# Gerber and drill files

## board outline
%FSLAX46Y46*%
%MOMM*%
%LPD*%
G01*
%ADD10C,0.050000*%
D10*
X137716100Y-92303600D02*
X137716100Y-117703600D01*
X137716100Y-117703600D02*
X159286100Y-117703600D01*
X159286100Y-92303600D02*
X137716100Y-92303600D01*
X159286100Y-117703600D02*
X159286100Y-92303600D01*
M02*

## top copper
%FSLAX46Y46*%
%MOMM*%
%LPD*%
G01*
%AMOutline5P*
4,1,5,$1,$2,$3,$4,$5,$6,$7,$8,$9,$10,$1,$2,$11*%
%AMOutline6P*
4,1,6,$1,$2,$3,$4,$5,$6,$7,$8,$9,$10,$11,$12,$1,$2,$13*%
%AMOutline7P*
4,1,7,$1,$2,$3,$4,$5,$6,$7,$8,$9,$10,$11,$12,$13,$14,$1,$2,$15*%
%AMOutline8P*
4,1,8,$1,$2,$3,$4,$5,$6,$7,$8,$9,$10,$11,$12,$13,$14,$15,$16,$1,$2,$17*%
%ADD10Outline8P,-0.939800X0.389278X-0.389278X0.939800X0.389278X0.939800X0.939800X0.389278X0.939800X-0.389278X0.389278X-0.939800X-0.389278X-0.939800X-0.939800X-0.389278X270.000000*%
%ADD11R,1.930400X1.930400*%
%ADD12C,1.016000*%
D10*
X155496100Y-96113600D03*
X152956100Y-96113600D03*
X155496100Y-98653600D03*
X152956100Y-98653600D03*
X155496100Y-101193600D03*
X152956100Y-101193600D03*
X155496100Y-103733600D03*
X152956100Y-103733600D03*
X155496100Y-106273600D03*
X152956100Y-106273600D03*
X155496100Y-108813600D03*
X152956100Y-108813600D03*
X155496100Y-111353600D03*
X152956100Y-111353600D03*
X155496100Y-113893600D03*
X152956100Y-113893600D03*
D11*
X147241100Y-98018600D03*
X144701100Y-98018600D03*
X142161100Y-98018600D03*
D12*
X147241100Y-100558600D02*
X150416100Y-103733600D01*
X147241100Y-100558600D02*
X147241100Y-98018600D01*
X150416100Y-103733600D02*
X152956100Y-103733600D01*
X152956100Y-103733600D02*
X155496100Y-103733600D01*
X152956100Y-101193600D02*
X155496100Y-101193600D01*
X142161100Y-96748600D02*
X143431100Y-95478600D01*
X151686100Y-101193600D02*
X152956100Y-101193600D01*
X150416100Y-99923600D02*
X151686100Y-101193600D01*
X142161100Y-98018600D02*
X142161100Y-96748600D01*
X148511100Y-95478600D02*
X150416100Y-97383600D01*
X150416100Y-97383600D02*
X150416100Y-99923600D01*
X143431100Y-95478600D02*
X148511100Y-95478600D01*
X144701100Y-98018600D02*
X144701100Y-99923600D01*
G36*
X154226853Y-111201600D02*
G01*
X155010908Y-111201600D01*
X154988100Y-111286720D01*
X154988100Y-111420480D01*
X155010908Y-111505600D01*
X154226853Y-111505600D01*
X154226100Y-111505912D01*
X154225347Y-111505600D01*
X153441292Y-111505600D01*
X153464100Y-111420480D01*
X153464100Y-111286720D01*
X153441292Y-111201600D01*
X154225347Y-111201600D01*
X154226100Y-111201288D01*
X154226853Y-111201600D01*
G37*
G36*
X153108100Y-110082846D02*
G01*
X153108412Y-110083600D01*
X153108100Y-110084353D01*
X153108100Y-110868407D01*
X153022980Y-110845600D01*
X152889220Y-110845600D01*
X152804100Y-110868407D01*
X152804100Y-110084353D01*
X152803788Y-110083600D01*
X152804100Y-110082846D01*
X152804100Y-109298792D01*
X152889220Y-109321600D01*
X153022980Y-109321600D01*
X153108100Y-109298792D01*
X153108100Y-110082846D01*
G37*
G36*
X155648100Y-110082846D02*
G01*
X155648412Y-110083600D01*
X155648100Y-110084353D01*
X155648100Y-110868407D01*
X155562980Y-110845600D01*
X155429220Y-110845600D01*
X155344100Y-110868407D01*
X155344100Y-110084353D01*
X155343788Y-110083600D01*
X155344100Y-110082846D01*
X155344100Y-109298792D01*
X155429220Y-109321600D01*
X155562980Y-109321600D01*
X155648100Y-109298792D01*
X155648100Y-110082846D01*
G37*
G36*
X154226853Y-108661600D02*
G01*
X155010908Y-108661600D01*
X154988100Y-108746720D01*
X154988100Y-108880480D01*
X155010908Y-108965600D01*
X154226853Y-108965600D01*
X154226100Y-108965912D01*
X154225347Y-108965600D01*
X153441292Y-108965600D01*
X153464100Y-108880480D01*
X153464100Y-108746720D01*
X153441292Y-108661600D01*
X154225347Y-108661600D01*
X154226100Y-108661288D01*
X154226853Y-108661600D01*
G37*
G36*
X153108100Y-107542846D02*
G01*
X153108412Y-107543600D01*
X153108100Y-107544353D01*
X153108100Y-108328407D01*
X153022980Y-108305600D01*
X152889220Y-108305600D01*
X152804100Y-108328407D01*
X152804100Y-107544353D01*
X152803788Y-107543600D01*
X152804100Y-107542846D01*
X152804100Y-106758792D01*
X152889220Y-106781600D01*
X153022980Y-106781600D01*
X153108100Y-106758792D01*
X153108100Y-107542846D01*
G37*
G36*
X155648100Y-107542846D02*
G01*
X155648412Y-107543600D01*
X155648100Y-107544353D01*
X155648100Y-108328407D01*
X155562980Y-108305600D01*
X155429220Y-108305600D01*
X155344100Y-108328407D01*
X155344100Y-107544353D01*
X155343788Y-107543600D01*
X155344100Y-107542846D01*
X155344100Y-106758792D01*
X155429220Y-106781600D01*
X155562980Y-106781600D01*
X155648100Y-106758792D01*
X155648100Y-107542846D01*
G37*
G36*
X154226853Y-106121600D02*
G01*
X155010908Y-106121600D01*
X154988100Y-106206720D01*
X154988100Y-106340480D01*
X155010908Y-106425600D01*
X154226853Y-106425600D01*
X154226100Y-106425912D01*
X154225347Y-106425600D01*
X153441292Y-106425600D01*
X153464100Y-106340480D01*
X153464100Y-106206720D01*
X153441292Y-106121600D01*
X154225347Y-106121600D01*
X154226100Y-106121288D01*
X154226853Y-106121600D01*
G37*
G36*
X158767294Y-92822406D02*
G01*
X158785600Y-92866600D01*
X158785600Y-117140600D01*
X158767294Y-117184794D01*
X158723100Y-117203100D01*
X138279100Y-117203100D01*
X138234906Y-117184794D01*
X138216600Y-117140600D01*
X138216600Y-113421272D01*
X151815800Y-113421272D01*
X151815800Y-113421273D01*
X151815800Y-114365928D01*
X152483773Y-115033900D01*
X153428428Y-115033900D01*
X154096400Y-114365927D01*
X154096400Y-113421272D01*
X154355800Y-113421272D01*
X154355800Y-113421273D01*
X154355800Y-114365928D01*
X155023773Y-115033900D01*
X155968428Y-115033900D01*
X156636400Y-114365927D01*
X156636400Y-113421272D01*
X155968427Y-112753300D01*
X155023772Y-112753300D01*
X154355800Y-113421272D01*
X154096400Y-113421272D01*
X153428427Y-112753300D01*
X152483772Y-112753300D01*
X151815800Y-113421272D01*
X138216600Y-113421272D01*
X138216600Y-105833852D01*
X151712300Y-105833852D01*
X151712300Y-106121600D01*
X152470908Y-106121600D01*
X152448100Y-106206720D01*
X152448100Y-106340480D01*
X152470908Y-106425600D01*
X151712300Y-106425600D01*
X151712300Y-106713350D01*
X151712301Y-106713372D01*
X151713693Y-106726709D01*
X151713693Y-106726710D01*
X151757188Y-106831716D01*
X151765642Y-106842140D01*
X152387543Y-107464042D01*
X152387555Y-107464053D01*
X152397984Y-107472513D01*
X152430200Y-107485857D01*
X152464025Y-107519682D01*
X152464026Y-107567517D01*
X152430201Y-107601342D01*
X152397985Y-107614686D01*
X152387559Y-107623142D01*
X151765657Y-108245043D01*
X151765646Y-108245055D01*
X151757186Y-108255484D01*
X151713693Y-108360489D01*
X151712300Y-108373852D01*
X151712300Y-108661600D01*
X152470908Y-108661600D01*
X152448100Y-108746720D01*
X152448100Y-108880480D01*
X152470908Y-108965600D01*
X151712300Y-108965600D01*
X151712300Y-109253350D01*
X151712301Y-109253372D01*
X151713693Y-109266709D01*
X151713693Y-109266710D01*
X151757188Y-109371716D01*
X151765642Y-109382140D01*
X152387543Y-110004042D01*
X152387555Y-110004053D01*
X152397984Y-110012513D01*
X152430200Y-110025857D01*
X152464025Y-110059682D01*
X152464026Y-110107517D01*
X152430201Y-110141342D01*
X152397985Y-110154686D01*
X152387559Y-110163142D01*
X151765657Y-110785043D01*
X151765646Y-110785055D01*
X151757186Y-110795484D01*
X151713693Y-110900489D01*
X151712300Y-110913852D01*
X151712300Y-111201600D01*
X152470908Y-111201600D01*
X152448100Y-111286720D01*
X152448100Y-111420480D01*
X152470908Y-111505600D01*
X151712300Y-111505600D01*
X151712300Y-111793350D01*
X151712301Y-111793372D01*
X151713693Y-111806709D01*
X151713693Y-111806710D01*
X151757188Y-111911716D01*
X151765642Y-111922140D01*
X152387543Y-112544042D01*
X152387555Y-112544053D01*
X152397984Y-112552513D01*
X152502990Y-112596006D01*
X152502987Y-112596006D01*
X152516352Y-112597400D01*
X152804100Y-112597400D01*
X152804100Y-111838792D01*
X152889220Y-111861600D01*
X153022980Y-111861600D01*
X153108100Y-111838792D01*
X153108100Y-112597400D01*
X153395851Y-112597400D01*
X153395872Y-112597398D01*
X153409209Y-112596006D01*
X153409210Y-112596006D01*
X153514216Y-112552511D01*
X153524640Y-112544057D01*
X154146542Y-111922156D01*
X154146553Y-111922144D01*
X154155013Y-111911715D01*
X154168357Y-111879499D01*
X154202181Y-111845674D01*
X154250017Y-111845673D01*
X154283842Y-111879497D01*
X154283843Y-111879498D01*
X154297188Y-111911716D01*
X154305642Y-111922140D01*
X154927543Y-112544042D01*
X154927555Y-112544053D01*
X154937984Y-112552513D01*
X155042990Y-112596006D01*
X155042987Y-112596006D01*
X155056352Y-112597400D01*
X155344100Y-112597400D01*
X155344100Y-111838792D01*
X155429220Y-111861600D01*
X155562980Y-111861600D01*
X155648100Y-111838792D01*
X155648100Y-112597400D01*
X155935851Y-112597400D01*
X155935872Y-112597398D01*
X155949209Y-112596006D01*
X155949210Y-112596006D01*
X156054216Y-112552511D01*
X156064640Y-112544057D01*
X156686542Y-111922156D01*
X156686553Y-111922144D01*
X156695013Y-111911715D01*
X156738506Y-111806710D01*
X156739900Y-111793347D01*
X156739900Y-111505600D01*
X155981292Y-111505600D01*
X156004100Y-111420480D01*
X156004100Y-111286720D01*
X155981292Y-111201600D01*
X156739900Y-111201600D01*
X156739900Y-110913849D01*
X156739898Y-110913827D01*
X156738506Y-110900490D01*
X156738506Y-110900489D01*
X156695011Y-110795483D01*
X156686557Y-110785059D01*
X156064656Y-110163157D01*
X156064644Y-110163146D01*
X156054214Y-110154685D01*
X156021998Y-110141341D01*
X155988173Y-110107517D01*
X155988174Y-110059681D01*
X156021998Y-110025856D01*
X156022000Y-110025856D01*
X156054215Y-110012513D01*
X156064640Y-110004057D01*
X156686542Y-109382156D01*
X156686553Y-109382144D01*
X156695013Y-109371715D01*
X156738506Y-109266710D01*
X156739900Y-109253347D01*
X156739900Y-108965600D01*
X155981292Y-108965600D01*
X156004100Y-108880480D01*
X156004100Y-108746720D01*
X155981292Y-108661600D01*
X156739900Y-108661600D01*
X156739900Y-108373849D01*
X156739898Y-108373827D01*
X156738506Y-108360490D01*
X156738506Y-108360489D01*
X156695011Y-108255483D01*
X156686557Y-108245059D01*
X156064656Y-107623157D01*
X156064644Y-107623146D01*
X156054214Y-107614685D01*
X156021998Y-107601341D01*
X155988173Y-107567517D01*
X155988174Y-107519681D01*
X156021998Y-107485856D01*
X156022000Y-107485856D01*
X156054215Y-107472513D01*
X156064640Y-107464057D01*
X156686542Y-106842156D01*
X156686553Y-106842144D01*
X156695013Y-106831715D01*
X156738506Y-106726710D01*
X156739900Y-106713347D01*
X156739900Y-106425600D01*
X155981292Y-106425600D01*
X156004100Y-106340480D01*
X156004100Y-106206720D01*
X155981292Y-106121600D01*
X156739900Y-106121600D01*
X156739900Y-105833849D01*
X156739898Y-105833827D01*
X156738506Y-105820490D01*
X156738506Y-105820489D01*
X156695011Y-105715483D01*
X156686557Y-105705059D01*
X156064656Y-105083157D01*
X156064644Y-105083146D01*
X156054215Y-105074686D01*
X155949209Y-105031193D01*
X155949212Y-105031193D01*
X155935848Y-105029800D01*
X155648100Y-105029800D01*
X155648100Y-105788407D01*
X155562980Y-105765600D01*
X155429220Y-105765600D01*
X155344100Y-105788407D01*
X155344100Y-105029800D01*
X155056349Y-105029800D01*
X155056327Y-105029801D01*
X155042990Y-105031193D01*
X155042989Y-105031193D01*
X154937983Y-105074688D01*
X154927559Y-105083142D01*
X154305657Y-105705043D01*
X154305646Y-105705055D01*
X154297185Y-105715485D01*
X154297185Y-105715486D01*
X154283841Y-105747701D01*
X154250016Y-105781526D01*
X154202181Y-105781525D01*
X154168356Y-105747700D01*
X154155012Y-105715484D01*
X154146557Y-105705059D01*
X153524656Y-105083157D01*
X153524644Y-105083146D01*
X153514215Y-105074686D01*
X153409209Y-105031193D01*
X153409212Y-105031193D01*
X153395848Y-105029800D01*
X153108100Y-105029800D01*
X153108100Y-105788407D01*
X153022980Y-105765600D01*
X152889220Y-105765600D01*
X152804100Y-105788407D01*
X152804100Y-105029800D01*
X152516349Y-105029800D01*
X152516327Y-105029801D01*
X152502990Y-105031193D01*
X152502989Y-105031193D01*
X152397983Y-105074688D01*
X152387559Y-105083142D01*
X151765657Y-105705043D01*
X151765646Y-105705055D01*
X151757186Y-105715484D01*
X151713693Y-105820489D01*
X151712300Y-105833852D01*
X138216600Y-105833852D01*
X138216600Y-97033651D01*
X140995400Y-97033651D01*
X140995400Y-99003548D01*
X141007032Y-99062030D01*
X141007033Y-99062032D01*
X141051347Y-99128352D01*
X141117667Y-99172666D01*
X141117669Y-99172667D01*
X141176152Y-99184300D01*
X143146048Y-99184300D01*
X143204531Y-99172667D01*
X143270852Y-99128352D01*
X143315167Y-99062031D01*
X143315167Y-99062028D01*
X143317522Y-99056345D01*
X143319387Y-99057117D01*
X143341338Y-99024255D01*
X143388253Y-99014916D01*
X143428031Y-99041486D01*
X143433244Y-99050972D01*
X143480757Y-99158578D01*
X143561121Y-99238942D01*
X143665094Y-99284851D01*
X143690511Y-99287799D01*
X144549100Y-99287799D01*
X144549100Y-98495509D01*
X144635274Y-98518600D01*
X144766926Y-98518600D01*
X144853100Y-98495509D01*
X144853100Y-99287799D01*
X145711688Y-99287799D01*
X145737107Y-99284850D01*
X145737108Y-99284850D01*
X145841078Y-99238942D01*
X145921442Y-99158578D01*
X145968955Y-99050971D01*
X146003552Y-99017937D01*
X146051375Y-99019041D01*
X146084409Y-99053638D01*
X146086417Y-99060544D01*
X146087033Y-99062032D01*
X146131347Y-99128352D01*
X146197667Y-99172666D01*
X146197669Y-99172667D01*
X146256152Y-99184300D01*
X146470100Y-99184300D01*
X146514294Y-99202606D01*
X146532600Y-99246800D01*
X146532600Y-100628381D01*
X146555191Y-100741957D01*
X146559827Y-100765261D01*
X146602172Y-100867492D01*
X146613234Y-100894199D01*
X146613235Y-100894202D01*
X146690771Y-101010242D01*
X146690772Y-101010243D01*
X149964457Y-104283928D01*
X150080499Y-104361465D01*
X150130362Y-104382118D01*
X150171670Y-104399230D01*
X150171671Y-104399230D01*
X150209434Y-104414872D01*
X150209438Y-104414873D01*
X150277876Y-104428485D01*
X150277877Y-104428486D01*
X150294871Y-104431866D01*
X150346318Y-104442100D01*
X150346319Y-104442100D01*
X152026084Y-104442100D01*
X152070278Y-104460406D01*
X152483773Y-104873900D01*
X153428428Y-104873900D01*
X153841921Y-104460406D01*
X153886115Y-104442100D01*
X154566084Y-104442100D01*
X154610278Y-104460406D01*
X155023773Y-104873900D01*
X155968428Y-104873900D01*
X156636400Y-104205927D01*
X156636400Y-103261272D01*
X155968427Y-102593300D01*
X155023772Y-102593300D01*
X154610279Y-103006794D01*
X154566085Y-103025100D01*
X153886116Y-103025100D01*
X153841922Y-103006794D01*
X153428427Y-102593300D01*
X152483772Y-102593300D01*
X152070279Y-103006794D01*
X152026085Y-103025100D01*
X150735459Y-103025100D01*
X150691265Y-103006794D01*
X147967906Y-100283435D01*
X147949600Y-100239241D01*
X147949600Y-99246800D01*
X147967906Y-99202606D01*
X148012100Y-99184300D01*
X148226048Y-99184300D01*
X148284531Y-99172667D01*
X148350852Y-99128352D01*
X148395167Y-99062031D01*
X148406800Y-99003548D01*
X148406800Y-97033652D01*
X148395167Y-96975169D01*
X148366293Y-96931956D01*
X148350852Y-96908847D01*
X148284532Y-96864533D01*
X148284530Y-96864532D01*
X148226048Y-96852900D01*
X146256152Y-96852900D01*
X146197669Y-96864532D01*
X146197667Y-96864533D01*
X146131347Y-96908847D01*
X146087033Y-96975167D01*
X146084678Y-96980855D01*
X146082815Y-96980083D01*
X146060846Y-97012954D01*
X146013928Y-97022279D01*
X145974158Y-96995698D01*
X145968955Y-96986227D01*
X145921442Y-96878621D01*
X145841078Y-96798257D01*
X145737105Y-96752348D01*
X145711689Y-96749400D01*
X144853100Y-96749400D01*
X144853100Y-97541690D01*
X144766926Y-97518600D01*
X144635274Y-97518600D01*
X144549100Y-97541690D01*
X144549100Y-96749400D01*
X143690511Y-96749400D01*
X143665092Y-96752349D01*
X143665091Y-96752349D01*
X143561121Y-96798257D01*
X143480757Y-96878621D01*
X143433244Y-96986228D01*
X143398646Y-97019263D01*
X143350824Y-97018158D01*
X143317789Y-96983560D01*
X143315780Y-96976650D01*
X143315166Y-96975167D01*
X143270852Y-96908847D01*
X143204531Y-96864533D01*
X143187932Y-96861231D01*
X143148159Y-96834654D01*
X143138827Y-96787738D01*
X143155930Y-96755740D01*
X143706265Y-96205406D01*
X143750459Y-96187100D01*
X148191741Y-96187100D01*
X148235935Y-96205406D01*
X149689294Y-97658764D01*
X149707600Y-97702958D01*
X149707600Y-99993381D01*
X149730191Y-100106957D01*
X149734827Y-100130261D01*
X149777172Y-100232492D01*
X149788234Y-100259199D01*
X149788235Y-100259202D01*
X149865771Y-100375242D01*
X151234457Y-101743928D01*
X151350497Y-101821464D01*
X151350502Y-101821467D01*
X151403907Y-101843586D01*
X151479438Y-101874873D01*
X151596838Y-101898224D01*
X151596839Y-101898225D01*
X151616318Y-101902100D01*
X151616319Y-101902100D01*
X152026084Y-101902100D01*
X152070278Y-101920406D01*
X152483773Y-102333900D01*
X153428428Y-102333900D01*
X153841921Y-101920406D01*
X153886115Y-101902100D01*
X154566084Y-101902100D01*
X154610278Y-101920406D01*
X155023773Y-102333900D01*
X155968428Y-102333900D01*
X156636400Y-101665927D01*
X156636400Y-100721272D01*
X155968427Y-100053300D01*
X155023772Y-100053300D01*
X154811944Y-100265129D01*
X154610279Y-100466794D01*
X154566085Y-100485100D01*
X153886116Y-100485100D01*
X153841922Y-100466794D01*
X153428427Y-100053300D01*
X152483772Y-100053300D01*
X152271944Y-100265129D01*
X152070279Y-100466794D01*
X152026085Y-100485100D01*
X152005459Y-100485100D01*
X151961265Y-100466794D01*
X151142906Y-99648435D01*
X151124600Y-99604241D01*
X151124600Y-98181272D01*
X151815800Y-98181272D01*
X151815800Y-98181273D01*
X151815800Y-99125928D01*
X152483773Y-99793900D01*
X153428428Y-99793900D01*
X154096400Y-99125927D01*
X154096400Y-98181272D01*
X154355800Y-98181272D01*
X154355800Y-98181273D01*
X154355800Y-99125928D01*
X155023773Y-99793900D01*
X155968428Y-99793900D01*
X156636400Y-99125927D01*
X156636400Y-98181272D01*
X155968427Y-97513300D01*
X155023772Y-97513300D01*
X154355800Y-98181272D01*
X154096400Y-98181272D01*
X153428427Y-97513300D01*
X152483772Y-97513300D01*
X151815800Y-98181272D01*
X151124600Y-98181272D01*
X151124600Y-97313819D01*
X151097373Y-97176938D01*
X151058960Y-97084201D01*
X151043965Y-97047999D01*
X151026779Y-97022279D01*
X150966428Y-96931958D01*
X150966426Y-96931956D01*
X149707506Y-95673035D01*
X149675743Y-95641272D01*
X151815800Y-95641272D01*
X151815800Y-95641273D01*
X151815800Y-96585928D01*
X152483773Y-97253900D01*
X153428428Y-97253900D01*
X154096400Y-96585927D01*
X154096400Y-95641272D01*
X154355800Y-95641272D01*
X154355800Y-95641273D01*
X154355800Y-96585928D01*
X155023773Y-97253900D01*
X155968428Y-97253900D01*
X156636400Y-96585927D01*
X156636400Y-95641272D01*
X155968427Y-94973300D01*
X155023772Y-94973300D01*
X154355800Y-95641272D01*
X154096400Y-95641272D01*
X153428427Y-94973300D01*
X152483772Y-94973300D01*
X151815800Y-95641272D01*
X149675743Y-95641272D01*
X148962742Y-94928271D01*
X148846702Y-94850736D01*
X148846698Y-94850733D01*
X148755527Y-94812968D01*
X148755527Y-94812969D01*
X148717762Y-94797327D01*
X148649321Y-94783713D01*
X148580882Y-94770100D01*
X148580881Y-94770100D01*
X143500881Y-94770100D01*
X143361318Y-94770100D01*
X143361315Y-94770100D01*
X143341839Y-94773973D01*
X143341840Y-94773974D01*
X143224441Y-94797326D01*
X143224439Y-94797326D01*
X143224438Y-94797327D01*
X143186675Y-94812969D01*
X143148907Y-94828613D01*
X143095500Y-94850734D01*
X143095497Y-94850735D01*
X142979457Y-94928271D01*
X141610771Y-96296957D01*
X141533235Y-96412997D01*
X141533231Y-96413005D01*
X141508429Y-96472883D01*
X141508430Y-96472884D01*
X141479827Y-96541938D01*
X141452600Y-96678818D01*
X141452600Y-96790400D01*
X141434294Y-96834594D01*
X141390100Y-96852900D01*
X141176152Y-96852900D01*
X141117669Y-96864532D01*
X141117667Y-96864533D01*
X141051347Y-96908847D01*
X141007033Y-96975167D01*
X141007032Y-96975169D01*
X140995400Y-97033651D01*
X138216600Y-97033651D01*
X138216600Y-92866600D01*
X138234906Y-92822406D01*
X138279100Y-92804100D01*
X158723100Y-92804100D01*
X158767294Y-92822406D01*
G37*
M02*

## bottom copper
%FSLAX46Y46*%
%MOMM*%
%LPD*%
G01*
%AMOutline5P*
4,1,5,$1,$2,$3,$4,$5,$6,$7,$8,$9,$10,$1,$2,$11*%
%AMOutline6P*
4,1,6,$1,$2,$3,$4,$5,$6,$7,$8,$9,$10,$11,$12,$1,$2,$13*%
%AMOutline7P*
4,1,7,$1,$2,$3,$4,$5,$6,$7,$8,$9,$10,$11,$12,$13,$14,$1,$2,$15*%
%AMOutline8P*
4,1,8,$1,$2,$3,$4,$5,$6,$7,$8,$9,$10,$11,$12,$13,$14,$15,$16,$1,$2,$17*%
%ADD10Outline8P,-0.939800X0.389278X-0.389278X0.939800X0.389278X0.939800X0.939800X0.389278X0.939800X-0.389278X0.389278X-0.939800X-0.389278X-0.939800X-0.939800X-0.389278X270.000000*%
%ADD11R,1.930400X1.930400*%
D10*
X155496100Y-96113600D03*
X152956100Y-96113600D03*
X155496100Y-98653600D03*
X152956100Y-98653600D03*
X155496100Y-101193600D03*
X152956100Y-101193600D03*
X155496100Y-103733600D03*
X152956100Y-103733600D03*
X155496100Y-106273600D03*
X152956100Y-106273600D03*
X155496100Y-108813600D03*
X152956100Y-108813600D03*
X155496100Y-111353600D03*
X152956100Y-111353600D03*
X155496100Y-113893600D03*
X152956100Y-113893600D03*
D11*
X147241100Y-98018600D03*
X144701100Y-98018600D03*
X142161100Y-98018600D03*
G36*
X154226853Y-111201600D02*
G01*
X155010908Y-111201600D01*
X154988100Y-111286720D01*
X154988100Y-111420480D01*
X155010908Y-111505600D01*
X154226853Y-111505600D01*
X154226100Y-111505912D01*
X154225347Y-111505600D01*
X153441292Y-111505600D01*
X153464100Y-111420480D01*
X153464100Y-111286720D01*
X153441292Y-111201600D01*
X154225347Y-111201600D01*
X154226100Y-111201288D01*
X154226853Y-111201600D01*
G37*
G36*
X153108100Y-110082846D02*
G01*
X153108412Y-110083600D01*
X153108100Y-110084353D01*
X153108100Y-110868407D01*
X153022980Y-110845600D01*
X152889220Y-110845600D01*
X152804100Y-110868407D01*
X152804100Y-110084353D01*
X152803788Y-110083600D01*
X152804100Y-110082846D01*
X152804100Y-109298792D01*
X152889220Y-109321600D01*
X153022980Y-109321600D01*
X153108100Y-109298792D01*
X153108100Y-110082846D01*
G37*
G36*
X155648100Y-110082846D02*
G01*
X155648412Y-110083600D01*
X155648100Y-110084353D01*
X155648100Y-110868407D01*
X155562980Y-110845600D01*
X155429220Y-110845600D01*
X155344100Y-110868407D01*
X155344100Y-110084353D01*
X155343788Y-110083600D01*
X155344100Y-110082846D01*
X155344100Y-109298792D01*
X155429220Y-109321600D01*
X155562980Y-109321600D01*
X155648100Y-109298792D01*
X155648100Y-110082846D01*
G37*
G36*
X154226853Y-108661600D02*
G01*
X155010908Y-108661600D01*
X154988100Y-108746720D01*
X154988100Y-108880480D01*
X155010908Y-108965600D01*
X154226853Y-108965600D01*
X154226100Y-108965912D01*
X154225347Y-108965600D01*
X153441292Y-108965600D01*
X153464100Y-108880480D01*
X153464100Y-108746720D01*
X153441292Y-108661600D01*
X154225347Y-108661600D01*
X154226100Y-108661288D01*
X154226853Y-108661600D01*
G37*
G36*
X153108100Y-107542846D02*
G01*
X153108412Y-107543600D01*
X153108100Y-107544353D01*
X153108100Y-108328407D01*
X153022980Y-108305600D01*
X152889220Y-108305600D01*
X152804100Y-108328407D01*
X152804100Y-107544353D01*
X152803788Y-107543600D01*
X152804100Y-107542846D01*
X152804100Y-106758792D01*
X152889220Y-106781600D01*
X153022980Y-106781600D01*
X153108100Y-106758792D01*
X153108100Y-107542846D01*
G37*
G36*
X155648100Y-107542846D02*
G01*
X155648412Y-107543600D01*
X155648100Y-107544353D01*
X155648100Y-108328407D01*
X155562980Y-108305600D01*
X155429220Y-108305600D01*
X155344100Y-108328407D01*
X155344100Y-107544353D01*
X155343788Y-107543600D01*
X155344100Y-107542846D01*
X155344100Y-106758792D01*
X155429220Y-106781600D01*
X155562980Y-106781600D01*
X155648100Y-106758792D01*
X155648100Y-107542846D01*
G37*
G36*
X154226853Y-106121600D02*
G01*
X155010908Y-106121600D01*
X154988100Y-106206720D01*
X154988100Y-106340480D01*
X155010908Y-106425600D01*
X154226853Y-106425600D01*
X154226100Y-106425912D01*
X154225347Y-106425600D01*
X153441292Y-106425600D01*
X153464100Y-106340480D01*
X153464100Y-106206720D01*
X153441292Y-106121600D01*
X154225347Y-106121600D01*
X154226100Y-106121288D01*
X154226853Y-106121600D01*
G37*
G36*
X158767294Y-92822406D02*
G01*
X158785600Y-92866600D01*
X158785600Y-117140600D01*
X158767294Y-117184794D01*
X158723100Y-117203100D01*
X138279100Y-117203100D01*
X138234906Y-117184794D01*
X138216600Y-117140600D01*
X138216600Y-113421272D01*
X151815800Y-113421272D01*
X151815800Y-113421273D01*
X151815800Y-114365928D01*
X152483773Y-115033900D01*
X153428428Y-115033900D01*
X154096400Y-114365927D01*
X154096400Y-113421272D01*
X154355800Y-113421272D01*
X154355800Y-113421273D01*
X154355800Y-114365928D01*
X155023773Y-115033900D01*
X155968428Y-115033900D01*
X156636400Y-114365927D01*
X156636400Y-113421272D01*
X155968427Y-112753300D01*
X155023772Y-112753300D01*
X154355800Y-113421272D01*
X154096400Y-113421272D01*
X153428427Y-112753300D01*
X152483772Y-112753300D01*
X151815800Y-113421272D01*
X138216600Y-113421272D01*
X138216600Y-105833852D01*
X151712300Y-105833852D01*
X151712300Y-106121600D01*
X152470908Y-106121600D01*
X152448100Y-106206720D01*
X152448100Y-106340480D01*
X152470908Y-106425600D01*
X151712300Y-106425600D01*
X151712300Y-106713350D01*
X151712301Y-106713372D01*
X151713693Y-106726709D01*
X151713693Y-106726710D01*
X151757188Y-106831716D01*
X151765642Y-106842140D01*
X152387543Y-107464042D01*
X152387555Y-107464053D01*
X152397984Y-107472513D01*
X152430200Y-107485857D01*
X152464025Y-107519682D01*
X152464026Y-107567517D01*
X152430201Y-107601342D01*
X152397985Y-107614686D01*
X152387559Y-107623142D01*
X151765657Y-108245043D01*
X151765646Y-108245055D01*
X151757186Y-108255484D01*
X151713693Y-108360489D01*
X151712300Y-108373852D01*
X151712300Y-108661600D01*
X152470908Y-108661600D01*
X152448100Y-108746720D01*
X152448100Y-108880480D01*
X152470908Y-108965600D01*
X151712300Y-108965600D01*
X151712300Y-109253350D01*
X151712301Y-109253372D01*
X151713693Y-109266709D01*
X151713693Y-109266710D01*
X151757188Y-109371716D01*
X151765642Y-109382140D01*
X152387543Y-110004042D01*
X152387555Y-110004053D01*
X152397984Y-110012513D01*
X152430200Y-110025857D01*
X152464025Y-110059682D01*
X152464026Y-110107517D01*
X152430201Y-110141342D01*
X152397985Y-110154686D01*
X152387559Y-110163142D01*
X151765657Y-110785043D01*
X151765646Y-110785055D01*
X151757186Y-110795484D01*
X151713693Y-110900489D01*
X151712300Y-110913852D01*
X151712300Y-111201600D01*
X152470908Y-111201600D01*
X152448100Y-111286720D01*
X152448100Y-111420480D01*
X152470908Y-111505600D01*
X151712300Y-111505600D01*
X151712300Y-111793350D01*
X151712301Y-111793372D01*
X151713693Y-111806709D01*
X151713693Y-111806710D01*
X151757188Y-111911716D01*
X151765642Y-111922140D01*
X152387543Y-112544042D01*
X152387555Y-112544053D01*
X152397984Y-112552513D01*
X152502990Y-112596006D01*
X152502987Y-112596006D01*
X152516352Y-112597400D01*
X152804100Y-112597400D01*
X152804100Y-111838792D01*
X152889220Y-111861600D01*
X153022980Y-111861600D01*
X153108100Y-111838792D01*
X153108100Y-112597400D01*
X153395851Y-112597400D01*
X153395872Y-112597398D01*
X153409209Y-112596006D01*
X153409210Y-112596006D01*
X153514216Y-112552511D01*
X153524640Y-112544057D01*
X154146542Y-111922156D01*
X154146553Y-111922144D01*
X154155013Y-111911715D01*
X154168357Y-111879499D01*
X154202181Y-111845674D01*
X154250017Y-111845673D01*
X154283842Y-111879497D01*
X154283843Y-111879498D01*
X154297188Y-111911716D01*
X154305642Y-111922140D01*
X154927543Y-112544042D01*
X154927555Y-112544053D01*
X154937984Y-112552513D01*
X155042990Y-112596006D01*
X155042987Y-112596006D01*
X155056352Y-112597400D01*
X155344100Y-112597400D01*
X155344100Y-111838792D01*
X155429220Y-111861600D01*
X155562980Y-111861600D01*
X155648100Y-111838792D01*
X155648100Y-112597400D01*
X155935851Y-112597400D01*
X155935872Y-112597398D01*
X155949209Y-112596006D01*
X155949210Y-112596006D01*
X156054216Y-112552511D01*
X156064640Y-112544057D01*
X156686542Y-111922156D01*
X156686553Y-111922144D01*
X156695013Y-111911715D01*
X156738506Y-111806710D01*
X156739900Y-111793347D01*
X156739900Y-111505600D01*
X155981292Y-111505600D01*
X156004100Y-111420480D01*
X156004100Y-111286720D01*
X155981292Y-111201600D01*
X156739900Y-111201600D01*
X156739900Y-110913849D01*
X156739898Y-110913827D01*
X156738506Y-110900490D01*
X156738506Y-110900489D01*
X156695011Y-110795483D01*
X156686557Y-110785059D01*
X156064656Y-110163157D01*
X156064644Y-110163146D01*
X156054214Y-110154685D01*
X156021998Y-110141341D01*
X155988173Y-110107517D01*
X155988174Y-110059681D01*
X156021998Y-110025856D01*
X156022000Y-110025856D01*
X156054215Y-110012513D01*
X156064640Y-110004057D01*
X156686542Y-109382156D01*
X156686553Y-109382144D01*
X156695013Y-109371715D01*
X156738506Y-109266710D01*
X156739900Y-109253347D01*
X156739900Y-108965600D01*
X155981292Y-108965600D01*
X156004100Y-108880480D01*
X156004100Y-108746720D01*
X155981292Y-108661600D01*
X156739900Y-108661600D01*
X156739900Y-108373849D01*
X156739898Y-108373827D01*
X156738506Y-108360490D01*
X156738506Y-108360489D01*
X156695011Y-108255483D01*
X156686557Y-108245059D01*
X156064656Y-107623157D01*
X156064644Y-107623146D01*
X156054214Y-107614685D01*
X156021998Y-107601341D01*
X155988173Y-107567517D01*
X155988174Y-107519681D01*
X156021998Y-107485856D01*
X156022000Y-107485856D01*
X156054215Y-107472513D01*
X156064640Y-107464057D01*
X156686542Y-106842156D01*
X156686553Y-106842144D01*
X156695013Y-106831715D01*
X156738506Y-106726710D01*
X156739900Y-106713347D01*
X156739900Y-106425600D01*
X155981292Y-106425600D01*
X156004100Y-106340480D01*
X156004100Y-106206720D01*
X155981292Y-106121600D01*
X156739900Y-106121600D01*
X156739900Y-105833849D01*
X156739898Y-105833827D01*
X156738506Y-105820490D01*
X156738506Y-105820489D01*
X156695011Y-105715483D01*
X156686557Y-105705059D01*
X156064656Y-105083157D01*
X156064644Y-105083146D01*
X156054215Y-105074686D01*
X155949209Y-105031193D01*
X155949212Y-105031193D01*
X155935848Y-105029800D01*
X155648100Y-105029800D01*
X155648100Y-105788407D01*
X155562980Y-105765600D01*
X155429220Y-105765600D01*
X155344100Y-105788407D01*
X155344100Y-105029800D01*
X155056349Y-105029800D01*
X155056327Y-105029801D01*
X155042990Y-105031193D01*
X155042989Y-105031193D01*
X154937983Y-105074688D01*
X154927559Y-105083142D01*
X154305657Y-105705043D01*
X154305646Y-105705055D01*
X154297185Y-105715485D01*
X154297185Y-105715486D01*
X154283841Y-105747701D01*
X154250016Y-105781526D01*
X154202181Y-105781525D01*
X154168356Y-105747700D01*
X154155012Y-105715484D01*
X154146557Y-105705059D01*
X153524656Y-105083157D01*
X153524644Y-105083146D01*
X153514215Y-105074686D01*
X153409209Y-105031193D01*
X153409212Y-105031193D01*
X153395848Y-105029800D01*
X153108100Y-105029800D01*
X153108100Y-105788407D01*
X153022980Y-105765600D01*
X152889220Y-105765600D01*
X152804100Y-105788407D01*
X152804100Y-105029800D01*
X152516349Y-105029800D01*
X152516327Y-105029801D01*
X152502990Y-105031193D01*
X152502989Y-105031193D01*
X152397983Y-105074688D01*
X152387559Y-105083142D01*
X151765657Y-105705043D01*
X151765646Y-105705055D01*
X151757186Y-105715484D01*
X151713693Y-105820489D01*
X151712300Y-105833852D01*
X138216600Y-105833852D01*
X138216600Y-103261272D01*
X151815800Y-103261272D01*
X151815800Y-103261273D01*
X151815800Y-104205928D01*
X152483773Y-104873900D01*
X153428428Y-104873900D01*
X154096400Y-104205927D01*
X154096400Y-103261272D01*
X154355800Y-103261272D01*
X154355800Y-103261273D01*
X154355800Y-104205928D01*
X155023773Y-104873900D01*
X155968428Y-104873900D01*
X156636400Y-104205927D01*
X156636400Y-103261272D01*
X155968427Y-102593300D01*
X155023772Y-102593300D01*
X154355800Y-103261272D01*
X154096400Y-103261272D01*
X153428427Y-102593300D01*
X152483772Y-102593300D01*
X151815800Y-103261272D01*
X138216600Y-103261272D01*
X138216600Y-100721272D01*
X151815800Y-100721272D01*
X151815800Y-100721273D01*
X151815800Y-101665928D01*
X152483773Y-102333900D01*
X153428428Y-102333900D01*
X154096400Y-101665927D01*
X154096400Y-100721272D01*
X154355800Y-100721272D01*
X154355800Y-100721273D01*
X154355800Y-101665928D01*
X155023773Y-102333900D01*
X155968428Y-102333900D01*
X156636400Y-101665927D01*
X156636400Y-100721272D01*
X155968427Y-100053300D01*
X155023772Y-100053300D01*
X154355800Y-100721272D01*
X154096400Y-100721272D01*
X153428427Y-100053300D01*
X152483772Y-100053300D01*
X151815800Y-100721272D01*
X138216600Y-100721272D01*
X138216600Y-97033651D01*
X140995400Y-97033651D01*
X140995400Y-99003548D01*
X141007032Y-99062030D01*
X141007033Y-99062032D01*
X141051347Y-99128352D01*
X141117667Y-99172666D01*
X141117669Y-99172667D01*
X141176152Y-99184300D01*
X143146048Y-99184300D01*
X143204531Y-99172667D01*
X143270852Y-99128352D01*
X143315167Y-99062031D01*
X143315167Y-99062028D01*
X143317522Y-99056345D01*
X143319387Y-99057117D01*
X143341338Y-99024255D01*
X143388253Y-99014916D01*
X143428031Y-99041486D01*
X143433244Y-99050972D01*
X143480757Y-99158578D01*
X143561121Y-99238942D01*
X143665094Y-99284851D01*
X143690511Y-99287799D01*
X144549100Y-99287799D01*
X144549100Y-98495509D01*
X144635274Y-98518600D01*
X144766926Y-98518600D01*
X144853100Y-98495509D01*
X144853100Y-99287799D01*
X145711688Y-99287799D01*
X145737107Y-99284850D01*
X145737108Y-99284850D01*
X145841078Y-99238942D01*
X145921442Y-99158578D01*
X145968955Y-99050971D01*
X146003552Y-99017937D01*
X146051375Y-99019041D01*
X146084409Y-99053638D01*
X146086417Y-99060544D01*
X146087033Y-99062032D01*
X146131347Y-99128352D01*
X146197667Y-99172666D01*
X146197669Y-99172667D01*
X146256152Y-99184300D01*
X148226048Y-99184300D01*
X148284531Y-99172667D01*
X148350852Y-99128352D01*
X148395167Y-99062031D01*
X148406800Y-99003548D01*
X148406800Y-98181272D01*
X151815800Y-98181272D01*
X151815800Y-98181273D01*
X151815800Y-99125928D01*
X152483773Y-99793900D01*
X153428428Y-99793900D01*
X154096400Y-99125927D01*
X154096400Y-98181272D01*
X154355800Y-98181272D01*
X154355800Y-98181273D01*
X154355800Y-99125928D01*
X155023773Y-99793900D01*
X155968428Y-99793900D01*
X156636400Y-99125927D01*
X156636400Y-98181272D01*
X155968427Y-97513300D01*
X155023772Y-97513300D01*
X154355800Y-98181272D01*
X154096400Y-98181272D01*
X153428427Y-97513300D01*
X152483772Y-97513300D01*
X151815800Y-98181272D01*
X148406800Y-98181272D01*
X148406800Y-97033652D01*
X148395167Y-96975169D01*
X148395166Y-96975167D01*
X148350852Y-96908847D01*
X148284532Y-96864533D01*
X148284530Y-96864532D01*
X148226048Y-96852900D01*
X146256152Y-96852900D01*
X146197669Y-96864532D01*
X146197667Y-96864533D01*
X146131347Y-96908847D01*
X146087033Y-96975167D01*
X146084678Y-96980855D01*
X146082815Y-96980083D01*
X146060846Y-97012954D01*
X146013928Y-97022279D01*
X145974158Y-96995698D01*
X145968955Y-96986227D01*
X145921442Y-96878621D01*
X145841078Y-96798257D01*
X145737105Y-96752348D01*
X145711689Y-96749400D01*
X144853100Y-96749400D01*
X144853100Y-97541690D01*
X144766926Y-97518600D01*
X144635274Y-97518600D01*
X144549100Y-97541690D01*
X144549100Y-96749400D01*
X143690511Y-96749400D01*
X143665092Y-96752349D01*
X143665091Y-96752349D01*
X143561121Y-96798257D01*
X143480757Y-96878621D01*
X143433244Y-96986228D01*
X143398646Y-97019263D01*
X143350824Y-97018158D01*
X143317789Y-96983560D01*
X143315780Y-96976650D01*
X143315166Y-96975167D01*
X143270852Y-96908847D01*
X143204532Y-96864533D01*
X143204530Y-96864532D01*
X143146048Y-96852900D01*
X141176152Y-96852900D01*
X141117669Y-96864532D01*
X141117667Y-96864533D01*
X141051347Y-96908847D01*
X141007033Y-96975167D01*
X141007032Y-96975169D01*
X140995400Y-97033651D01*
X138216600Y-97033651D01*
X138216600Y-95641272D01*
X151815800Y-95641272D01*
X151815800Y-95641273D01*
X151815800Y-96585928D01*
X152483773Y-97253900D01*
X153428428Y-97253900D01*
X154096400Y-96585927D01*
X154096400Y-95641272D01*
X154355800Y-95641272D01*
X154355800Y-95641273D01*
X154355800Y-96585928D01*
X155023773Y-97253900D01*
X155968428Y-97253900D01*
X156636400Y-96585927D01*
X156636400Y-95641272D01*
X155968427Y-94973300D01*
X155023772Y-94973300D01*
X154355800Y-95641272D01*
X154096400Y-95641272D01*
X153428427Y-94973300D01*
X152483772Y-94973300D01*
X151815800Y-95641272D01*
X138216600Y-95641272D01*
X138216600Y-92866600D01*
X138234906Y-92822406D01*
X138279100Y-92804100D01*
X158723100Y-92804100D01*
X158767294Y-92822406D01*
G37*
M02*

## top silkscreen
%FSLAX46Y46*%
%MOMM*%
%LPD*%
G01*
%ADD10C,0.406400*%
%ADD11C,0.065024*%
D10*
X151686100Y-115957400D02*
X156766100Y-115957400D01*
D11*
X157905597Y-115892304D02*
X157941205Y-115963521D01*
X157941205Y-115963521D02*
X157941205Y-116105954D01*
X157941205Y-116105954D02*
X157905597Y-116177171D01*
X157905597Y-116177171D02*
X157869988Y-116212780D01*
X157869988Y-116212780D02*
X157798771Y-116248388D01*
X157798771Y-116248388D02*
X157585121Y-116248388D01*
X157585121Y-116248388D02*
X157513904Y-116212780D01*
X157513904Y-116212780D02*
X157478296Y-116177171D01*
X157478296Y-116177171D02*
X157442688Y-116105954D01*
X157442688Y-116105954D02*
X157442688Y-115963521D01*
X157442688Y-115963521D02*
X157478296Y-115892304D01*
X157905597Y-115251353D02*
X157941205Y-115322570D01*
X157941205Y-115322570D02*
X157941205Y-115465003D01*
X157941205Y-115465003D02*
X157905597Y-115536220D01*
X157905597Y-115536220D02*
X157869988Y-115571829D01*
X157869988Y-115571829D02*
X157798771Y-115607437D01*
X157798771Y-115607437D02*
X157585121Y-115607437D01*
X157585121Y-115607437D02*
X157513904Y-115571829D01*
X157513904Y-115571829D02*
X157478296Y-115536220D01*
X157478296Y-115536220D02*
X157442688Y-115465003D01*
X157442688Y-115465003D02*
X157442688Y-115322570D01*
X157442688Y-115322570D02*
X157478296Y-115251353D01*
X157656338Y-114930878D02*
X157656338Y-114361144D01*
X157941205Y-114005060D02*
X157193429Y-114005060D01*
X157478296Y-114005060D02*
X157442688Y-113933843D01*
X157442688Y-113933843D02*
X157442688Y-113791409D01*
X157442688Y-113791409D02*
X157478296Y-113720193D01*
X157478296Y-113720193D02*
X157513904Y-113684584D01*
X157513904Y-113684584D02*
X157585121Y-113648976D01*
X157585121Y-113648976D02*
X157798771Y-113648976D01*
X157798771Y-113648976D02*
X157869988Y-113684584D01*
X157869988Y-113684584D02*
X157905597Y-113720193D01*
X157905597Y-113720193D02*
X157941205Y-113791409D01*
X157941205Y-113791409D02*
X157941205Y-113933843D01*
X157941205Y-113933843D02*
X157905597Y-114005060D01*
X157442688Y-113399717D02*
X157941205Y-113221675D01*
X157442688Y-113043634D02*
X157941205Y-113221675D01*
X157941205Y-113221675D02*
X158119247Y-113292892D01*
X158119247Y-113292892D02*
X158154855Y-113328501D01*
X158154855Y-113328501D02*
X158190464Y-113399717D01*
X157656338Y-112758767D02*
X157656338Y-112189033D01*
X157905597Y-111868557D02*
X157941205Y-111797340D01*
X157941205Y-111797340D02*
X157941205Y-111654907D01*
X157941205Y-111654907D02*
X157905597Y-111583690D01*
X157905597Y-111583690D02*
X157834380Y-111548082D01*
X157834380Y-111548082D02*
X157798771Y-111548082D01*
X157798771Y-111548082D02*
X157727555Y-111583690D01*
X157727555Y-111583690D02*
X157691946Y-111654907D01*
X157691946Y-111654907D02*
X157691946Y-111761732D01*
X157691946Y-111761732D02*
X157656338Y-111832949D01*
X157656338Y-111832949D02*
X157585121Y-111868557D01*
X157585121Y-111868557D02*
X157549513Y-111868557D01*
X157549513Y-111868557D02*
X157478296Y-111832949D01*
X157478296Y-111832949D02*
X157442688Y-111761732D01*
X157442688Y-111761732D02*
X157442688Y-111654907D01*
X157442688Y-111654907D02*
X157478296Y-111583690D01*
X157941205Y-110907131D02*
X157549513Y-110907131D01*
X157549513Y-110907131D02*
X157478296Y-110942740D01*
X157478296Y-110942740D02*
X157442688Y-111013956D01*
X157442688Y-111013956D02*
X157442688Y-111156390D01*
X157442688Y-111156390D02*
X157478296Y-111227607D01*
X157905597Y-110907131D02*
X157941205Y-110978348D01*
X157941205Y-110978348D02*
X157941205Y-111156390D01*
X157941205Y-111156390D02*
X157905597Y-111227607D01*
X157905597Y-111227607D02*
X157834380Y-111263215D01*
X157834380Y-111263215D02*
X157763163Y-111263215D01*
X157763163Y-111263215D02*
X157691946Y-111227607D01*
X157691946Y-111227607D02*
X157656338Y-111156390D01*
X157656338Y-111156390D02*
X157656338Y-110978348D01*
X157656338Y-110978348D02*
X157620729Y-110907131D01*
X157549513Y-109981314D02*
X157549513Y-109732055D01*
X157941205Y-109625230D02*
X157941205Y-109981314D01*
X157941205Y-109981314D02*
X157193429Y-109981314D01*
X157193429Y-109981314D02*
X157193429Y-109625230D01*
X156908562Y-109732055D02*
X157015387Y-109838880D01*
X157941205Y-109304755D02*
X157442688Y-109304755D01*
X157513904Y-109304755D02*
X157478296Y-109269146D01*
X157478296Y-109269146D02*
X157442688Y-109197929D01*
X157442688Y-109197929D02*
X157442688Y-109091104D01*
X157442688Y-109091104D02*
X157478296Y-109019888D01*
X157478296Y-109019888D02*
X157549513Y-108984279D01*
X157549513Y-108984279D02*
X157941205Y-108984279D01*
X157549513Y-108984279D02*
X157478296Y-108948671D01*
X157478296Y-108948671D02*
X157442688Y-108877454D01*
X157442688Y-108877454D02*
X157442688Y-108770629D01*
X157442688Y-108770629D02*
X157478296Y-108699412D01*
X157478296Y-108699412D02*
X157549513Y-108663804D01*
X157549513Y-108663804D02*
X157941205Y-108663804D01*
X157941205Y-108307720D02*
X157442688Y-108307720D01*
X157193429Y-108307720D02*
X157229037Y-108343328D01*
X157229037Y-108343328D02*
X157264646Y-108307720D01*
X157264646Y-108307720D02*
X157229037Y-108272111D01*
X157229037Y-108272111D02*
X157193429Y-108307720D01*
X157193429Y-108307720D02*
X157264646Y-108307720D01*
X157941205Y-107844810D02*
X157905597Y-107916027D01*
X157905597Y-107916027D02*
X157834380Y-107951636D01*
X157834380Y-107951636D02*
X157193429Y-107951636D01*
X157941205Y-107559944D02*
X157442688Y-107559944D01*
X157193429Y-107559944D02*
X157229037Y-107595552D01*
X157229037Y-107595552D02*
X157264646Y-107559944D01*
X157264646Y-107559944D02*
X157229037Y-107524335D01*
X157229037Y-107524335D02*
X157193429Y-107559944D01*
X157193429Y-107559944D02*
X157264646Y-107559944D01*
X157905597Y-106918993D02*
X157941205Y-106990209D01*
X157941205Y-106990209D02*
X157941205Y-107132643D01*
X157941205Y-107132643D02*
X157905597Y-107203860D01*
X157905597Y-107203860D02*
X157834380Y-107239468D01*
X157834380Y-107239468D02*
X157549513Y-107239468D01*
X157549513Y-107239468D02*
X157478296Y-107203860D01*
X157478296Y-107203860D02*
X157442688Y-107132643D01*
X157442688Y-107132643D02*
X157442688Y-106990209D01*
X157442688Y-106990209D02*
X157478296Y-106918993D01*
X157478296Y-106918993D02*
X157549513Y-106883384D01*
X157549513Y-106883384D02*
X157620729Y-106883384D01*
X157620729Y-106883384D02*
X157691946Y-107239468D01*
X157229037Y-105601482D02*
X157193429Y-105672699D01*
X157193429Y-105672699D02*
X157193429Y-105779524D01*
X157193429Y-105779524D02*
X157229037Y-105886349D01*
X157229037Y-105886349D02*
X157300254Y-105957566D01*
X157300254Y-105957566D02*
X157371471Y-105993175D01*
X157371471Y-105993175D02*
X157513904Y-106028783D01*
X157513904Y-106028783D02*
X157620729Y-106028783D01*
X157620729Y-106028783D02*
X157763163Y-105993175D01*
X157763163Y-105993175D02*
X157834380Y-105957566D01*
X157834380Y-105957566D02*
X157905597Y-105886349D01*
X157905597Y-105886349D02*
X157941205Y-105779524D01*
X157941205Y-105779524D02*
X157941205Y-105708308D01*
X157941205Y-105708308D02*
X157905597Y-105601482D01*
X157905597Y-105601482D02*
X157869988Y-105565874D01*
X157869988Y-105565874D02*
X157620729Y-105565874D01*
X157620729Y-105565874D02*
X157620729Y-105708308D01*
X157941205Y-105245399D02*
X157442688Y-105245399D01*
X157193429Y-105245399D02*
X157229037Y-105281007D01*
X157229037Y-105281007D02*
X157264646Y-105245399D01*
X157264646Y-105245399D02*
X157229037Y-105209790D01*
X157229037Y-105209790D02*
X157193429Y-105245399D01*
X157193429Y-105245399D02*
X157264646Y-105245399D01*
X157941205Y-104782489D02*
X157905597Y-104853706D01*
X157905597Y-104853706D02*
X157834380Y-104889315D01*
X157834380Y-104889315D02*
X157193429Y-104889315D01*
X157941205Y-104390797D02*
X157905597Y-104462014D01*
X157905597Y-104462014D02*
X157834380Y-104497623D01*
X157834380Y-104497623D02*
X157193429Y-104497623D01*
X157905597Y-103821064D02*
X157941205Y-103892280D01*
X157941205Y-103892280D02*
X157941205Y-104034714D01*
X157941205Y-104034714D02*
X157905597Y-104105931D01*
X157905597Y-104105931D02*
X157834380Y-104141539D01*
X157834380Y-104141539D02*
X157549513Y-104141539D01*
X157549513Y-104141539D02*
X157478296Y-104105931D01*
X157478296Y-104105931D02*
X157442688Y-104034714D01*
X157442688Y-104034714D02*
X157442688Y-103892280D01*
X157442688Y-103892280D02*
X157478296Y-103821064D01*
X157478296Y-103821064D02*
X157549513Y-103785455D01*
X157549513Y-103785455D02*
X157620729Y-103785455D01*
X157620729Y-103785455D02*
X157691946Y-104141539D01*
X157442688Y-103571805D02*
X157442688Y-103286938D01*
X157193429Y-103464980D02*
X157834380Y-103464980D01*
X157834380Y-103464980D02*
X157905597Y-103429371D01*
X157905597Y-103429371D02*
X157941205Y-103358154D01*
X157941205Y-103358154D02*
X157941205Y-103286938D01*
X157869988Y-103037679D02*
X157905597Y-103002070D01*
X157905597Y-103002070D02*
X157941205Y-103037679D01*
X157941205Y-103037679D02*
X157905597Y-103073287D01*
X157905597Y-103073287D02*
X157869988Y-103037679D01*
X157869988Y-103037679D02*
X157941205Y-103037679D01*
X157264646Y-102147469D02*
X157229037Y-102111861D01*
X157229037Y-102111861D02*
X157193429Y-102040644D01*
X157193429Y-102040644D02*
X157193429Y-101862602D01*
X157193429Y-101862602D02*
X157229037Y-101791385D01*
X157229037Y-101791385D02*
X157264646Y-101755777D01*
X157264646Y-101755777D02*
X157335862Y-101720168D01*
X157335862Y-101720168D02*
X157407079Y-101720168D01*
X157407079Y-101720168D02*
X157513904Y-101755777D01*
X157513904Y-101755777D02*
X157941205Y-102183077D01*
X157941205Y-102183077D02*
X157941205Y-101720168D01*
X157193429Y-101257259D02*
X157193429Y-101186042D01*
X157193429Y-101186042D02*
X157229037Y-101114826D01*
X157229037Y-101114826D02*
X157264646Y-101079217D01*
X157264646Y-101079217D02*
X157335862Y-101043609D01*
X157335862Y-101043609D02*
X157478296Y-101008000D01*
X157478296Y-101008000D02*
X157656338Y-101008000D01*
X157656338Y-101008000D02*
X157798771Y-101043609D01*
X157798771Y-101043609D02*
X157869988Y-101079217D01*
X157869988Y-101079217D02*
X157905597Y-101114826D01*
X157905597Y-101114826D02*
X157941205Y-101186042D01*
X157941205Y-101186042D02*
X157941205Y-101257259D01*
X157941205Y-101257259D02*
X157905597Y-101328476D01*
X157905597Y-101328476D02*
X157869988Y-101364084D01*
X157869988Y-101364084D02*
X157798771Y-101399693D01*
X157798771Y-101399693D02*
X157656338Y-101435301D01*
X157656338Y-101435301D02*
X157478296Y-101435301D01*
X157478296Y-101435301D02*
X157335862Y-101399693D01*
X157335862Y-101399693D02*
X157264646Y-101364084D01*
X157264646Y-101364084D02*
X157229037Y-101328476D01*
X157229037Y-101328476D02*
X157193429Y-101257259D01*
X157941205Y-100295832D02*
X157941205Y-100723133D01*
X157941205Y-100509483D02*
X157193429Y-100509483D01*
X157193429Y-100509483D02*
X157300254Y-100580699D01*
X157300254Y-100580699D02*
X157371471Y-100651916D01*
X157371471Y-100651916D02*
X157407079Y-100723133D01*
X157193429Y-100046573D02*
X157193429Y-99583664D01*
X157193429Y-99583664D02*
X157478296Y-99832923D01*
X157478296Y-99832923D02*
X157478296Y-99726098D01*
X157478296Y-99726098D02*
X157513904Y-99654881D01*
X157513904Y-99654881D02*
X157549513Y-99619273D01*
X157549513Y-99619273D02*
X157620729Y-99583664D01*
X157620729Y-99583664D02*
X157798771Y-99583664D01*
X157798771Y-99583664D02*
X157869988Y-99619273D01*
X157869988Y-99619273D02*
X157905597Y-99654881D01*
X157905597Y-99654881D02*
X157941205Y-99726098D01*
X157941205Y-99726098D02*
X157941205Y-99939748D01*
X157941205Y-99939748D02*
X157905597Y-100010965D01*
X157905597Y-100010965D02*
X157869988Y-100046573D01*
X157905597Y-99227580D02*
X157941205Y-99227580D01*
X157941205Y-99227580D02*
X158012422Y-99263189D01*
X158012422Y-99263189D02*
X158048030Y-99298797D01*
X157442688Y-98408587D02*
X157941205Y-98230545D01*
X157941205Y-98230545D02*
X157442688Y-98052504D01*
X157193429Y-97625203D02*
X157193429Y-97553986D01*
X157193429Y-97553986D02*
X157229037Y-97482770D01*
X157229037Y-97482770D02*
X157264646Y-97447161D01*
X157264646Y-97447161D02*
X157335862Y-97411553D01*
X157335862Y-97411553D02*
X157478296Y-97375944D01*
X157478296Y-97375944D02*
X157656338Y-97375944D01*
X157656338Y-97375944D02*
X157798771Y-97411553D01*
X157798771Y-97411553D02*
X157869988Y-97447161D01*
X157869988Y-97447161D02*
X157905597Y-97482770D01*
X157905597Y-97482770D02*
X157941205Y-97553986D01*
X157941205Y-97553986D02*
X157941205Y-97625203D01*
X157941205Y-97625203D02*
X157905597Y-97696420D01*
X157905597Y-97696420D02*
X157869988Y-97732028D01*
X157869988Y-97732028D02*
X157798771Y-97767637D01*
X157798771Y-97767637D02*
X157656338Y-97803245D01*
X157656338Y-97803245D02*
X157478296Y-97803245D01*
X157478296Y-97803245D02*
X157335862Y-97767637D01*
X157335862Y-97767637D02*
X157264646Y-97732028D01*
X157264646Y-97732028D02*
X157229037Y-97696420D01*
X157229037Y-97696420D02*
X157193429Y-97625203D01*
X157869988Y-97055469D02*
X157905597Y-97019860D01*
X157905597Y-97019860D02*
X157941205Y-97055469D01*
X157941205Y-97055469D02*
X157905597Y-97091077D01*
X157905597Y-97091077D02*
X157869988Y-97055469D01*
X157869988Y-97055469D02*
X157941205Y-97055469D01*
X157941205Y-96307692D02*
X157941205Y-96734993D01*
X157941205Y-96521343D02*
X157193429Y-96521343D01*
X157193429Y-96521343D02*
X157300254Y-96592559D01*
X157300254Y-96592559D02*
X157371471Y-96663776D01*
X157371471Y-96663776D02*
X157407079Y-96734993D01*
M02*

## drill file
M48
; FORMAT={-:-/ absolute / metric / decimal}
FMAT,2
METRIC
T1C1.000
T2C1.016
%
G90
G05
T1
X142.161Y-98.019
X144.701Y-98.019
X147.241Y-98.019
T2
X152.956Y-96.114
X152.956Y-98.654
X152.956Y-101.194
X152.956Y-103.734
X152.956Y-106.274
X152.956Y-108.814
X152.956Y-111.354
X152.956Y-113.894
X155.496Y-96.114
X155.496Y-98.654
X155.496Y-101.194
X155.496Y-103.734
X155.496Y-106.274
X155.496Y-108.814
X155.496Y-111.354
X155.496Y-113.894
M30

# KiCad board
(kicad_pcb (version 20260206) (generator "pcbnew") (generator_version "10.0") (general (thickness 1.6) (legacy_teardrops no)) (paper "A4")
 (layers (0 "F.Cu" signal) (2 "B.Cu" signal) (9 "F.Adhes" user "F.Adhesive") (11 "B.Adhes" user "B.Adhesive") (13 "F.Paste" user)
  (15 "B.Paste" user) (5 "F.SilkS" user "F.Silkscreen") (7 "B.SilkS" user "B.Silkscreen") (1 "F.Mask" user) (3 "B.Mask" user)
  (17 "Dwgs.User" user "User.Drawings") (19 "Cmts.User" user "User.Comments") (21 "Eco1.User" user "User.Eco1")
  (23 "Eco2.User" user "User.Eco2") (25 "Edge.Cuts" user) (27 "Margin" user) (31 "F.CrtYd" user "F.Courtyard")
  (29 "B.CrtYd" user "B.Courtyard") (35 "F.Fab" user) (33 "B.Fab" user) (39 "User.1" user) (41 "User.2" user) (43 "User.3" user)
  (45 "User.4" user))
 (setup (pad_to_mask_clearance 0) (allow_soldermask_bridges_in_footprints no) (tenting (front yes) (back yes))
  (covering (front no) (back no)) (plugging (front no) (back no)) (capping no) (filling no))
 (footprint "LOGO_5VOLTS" (layer "F.Cu") (at 138.8273 117.2274)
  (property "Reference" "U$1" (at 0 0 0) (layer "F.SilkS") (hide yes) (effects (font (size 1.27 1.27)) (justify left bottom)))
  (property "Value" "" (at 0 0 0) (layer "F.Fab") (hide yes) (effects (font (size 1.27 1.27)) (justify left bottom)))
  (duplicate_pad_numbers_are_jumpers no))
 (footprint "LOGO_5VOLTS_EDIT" (layer "F.Cu") (at 139.6211 106.2736)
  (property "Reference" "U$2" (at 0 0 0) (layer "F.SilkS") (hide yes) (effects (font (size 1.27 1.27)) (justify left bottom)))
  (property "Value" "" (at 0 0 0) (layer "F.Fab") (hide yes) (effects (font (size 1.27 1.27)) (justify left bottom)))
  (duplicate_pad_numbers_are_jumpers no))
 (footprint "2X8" (layer "B.Cu") (at 155.4961 96.1136 -90)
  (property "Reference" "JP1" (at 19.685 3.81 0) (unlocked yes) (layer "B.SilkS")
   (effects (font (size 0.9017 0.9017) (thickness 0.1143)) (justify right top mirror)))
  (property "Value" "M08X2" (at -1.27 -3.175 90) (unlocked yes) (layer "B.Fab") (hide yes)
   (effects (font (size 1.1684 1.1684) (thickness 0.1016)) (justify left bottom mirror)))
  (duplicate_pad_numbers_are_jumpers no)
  (pad "1" thru_hole roundrect (at 0 0 270) (size 1.8796 1.8796) (drill 1.016) (layers "*.Cu" "*.Mask") (remove_unused_layers no)
   (roundrect_rratio 0.25) (chamfer_ratio 0.2928932188) (chamfer top_left top_right bottom_left bottom_right) (solder_mask_margin 0.0762)
   (thermal_bridge_angle 0))
  (pad "2" thru_hole roundrect (at 0 2.54 270) (size 1.8796 1.8796) (drill 1.016) (layers "*.Cu" "*.Mask") (remove_unused_layers no)
   (roundrect_rratio 0.25) (chamfer_ratio 0.2928932188) (chamfer top_left top_right bottom_left bottom_right) (solder_mask_margin 0.0762)
   (thermal_bridge_angle 0))
  (pad "3" thru_hole roundrect (at 2.54 0 270) (size 1.8796 1.8796) (drill 1.016) (layers "*.Cu" "*.Mask") (remove_unused_layers no)
   (roundrect_rratio 0.25) (chamfer_ratio 0.2928932188) (chamfer top_left top_right bottom_left bottom_right) (solder_mask_margin 0.0762)
   (thermal_bridge_angle 0))
  (pad "4" thru_hole roundrect (at 2.54 2.54 270) (size 1.8796 1.8796) (drill 1.016) (layers "*.Cu" "*.Mask") (remove_unused_layers no)
   (roundrect_rratio 0.25) (chamfer_ratio 0.2928932188) (chamfer top_left top_right bottom_left bottom_right) (solder_mask_margin 0.0762)
   (thermal_bridge_angle 0))
  (pad "5" thru_hole roundrect (at 5.08 0 270) (size 1.8796 1.8796) (drill 1.016) (layers "*.Cu" "*.Mask") (remove_unused_layers no)
   (roundrect_rratio 0.25) (chamfer_ratio 0.2928932188) (chamfer top_left top_right bottom_left bottom_right) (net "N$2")
   (solder_mask_margin 0.0762) (thermal_bridge_angle 0))
  (pad "6" thru_hole roundrect (at 5.08 2.54 270) (size 1.8796 1.8796) (drill 1.016) (layers "*.Cu" "*.Mask") (remove_unused_layers no)
   (roundrect_rratio 0.25) (chamfer_ratio 0.2928932188) (chamfer top_left top_right bottom_left bottom_right) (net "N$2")
   (solder_mask_margin 0.0762) (thermal_bridge_angle 0))
  (pad "7" thru_hole roundrect (at 7.62 0 270) (size 1.8796 1.8796) (drill 1.016) (layers "*.Cu" "*.Mask") (remove_unused_layers no)
   (roundrect_rratio 0.25) (chamfer_ratio 0.2928932188) (chamfer top_left top_right bottom_left bottom_right) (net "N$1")
   (solder_mask_margin 0.0762) (thermal_bridge_angle 0))
  (pad "8" thru_hole roundrect (at 7.62 2.54 270) (size 1.8796 1.8796) (drill 1.016) (layers "*.Cu" "*.Mask") (remove_unused_layers no)
   (roundrect_rratio 0.25) (chamfer_ratio 0.2928932188) (chamfer top_left top_right bottom_left bottom_right) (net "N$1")
   (solder_mask_margin 0.0762) (thermal_bridge_angle 0))
  (pad "9" thru_hole roundrect (at 10.16 0 270) (size 1.8796 1.8796) (drill 1.016) (layers "*.Cu" "*.Mask") (remove_unused_layers no)
   (roundrect_rratio 0.25) (chamfer_ratio 0.2928932188) (chamfer top_left top_right bottom_left bottom_right) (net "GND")
   (solder_mask_margin 0.0762) (thermal_bridge_angle 0))
  (pad "10" thru_hole roundrect (at 10.16 2.54 270) (size 1.8796 1.8796) (drill 1.016) (layers "*.Cu" "*.Mask") (remove_unused_layers no)
   (roundrect_rratio 0.25) (chamfer_ratio 0.2928932188) (chamfer top_left top_right bottom_left bottom_right) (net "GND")
   (solder_mask_margin 0.0762) (thermal_bridge_angle 0))
  (pad "11" thru_hole roundrect (at 12.7 0 270) (size 1.8796 1.8796) (drill 1.016) (layers "*.Cu" "*.Mask") (remove_unused_layers no)
   (roundrect_rratio 0.25) (chamfer_ratio 0.2928932188) (chamfer top_left top_right bottom_left bottom_right) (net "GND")
   (solder_mask_margin 0.0762) (thermal_bridge_angle 0))
  (pad "12" thru_hole roundrect (at 12.7 2.54 270) (size 1.8796 1.8796) (drill 1.016) (layers "*.Cu" "*.Mask") (remove_unused_layers no)
   (roundrect_rratio 0.25) (chamfer_ratio 0.2928932188) (chamfer top_left top_right bottom_left bottom_right) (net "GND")
   (solder_mask_margin 0.0762) (thermal_bridge_angle 0))
  (pad "13" thru_hole roundrect (at 15.24 0 270) (size 1.8796 1.8796) (drill 1.016) (layers "*.Cu" "*.Mask") (remove_unused_layers no)
   (roundrect_rratio 0.25) (chamfer_ratio 0.2928932188) (chamfer top_left top_right bottom_left bottom_right) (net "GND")
   (solder_mask_margin 0.0762) (thermal_bridge_angle 0))
  (pad "14" thru_hole roundrect (at 15.24 2.54 270) (size 1.8796 1.8796) (drill 1.016) (layers "*.Cu" "*.Mask") (remove_unused_layers no)
   (roundrect_rratio 0.25) (chamfer_ratio 0.2928932188) (chamfer top_left top_right bottom_left bottom_right) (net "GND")
   (solder_mask_margin 0.0762) (thermal_bridge_angle 0))
  (pad "15" thru_hole roundrect (at 17.78 0 270) (size 1.8796 1.8796) (drill 1.016) (layers "*.Cu" "*.Mask") (remove_unused_layers no)
   (roundrect_rratio 0.25) (chamfer_ratio 0.2928932188) (chamfer top_left top_right bottom_left bottom_right) (solder_mask_margin 0.0762)
   (thermal_bridge_angle 0))
  (pad "16" thru_hole roundrect (at 17.78 2.54 270) (size 1.8796 1.8796) (drill 1.016) (layers "*.Cu" "*.Mask") (remove_unused_layers no)
   (roundrect_rratio 0.25) (chamfer_ratio 0.2928932188) (chamfer top_left top_right bottom_left bottom_right) (solder_mask_margin 0.0762)
   (thermal_bridge_angle 0)))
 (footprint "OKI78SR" (layer "B.Cu") (at 144.7011 98.0186)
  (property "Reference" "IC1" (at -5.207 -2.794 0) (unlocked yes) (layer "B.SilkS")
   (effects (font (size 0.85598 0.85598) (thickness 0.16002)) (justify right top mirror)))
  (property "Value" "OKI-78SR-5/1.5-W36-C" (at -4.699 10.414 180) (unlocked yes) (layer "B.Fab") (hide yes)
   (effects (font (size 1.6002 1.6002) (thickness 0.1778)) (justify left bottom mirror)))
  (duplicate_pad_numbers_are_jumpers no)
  (pad "1" thru_hole rect (at 2.54 0 270) (size 1.9304 1.9304) (drill 1) (layers "*.Cu" "*.Mask") (remove_unused_layers no) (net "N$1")
   (solder_mask_margin 0.0762) (thermal_bridge_angle 0))
  (pad "2" thru_hole rect (at 0 0 270) (size 1.9304 1.9304) (drill 1) (layers "*.Cu" "*.Mask") (remove_unused_layers no) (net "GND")
   (solder_mask_margin 0.0762) (thermal_bridge_angle 0))
  (pad "3" thru_hole rect (at -2.54 0 270) (size 1.9304 1.9304) (drill 1) (layers "*.Cu" "*.Mask") (remove_unused_layers no) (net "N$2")
   (solder_mask_margin 0.0762) (thermal_bridge_angle 0)))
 (gr_line (start 151.6861 115.9574) (end 156.7661 115.9574) (stroke (width 0.4064) (type solid)) (layer "F.SilkS"))
 (gr_line (start 137.7161 92.3036) (end 137.7161 117.7036) (stroke (width 0.05) (type solid)) (layer "Edge.Cuts"))
 (gr_line (start 137.7161 117.7036) (end 159.2861 117.7036) (stroke (width 0.05) (type solid)) (layer "Edge.Cuts"))
 (gr_line (start 159.2861 92.3036) (end 137.7161 92.3036) (stroke (width 0.05) (type solid)) (layer "Edge.Cuts"))
 (gr_line (start 159.2861 117.7036) (end 159.2861 92.3036) (stroke (width 0.05) (type solid)) (layer "Edge.Cuts"))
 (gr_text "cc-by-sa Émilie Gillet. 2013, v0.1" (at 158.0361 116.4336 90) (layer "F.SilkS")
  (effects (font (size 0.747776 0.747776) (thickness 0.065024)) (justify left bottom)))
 (segment (start 147.2411 100.5586) (end 150.4161 103.7336) (width 1.016) (layer "F.Cu") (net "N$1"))
 (segment (start 147.2411 100.5586) (end 147.2411 98.0186) (width 1.016) (layer "F.Cu") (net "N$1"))
 (segment (start 150.4161 103.7336) (end 152.9561 103.7336) (width 1.016) (layer "F.Cu") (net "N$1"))
 (segment (start 152.9561 103.7336) (end 155.4961 103.7336) (width 1.016) (layer "F.Cu") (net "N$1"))
 (segment (start 152.9561 101.1936) (end 155.4961 101.1936) (width 1.016) (layer "F.Cu") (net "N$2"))
 (segment (start 142.1611 96.7486) (end 143.4311 95.4786) (width 1.016) (layer "F.Cu") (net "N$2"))
 (segment (start 151.6861 101.1936) (end 152.9561 101.1936) (width 1.016) (layer "F.Cu") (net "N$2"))
 (segment (start 150.4161 99.9236) (end 151.6861 101.1936) (width 1.016) (layer "F.Cu") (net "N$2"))
 (segment (start 142.1611 98.0186) (end 142.1611 96.7486) (width 1.016) (layer "F.Cu") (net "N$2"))
 (segment (start 148.5111 95.4786) (end 150.4161 97.3836) (width 1.016) (layer "F.Cu") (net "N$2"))
 (segment (start 150.4161 97.3836) (end 150.4161 99.9236) (width 1.016) (layer "F.Cu") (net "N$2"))
 (segment (start 143.4311 95.4786) (end 148.5111 95.4786) (width 1.016) (layer "F.Cu") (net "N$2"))
 (segment (start 144.7011 98.0186) (end 144.7011 99.9236) (width 1.016) (layer "F.Cu") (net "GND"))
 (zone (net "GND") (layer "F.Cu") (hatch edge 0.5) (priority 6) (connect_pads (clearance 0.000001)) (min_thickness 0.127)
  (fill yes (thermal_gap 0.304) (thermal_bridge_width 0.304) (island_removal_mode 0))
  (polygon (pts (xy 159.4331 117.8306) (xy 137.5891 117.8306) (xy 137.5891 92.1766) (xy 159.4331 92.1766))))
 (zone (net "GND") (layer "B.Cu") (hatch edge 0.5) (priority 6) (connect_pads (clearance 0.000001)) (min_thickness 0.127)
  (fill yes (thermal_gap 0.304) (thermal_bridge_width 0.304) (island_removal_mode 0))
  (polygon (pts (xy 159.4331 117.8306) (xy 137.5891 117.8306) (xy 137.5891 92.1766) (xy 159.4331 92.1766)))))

